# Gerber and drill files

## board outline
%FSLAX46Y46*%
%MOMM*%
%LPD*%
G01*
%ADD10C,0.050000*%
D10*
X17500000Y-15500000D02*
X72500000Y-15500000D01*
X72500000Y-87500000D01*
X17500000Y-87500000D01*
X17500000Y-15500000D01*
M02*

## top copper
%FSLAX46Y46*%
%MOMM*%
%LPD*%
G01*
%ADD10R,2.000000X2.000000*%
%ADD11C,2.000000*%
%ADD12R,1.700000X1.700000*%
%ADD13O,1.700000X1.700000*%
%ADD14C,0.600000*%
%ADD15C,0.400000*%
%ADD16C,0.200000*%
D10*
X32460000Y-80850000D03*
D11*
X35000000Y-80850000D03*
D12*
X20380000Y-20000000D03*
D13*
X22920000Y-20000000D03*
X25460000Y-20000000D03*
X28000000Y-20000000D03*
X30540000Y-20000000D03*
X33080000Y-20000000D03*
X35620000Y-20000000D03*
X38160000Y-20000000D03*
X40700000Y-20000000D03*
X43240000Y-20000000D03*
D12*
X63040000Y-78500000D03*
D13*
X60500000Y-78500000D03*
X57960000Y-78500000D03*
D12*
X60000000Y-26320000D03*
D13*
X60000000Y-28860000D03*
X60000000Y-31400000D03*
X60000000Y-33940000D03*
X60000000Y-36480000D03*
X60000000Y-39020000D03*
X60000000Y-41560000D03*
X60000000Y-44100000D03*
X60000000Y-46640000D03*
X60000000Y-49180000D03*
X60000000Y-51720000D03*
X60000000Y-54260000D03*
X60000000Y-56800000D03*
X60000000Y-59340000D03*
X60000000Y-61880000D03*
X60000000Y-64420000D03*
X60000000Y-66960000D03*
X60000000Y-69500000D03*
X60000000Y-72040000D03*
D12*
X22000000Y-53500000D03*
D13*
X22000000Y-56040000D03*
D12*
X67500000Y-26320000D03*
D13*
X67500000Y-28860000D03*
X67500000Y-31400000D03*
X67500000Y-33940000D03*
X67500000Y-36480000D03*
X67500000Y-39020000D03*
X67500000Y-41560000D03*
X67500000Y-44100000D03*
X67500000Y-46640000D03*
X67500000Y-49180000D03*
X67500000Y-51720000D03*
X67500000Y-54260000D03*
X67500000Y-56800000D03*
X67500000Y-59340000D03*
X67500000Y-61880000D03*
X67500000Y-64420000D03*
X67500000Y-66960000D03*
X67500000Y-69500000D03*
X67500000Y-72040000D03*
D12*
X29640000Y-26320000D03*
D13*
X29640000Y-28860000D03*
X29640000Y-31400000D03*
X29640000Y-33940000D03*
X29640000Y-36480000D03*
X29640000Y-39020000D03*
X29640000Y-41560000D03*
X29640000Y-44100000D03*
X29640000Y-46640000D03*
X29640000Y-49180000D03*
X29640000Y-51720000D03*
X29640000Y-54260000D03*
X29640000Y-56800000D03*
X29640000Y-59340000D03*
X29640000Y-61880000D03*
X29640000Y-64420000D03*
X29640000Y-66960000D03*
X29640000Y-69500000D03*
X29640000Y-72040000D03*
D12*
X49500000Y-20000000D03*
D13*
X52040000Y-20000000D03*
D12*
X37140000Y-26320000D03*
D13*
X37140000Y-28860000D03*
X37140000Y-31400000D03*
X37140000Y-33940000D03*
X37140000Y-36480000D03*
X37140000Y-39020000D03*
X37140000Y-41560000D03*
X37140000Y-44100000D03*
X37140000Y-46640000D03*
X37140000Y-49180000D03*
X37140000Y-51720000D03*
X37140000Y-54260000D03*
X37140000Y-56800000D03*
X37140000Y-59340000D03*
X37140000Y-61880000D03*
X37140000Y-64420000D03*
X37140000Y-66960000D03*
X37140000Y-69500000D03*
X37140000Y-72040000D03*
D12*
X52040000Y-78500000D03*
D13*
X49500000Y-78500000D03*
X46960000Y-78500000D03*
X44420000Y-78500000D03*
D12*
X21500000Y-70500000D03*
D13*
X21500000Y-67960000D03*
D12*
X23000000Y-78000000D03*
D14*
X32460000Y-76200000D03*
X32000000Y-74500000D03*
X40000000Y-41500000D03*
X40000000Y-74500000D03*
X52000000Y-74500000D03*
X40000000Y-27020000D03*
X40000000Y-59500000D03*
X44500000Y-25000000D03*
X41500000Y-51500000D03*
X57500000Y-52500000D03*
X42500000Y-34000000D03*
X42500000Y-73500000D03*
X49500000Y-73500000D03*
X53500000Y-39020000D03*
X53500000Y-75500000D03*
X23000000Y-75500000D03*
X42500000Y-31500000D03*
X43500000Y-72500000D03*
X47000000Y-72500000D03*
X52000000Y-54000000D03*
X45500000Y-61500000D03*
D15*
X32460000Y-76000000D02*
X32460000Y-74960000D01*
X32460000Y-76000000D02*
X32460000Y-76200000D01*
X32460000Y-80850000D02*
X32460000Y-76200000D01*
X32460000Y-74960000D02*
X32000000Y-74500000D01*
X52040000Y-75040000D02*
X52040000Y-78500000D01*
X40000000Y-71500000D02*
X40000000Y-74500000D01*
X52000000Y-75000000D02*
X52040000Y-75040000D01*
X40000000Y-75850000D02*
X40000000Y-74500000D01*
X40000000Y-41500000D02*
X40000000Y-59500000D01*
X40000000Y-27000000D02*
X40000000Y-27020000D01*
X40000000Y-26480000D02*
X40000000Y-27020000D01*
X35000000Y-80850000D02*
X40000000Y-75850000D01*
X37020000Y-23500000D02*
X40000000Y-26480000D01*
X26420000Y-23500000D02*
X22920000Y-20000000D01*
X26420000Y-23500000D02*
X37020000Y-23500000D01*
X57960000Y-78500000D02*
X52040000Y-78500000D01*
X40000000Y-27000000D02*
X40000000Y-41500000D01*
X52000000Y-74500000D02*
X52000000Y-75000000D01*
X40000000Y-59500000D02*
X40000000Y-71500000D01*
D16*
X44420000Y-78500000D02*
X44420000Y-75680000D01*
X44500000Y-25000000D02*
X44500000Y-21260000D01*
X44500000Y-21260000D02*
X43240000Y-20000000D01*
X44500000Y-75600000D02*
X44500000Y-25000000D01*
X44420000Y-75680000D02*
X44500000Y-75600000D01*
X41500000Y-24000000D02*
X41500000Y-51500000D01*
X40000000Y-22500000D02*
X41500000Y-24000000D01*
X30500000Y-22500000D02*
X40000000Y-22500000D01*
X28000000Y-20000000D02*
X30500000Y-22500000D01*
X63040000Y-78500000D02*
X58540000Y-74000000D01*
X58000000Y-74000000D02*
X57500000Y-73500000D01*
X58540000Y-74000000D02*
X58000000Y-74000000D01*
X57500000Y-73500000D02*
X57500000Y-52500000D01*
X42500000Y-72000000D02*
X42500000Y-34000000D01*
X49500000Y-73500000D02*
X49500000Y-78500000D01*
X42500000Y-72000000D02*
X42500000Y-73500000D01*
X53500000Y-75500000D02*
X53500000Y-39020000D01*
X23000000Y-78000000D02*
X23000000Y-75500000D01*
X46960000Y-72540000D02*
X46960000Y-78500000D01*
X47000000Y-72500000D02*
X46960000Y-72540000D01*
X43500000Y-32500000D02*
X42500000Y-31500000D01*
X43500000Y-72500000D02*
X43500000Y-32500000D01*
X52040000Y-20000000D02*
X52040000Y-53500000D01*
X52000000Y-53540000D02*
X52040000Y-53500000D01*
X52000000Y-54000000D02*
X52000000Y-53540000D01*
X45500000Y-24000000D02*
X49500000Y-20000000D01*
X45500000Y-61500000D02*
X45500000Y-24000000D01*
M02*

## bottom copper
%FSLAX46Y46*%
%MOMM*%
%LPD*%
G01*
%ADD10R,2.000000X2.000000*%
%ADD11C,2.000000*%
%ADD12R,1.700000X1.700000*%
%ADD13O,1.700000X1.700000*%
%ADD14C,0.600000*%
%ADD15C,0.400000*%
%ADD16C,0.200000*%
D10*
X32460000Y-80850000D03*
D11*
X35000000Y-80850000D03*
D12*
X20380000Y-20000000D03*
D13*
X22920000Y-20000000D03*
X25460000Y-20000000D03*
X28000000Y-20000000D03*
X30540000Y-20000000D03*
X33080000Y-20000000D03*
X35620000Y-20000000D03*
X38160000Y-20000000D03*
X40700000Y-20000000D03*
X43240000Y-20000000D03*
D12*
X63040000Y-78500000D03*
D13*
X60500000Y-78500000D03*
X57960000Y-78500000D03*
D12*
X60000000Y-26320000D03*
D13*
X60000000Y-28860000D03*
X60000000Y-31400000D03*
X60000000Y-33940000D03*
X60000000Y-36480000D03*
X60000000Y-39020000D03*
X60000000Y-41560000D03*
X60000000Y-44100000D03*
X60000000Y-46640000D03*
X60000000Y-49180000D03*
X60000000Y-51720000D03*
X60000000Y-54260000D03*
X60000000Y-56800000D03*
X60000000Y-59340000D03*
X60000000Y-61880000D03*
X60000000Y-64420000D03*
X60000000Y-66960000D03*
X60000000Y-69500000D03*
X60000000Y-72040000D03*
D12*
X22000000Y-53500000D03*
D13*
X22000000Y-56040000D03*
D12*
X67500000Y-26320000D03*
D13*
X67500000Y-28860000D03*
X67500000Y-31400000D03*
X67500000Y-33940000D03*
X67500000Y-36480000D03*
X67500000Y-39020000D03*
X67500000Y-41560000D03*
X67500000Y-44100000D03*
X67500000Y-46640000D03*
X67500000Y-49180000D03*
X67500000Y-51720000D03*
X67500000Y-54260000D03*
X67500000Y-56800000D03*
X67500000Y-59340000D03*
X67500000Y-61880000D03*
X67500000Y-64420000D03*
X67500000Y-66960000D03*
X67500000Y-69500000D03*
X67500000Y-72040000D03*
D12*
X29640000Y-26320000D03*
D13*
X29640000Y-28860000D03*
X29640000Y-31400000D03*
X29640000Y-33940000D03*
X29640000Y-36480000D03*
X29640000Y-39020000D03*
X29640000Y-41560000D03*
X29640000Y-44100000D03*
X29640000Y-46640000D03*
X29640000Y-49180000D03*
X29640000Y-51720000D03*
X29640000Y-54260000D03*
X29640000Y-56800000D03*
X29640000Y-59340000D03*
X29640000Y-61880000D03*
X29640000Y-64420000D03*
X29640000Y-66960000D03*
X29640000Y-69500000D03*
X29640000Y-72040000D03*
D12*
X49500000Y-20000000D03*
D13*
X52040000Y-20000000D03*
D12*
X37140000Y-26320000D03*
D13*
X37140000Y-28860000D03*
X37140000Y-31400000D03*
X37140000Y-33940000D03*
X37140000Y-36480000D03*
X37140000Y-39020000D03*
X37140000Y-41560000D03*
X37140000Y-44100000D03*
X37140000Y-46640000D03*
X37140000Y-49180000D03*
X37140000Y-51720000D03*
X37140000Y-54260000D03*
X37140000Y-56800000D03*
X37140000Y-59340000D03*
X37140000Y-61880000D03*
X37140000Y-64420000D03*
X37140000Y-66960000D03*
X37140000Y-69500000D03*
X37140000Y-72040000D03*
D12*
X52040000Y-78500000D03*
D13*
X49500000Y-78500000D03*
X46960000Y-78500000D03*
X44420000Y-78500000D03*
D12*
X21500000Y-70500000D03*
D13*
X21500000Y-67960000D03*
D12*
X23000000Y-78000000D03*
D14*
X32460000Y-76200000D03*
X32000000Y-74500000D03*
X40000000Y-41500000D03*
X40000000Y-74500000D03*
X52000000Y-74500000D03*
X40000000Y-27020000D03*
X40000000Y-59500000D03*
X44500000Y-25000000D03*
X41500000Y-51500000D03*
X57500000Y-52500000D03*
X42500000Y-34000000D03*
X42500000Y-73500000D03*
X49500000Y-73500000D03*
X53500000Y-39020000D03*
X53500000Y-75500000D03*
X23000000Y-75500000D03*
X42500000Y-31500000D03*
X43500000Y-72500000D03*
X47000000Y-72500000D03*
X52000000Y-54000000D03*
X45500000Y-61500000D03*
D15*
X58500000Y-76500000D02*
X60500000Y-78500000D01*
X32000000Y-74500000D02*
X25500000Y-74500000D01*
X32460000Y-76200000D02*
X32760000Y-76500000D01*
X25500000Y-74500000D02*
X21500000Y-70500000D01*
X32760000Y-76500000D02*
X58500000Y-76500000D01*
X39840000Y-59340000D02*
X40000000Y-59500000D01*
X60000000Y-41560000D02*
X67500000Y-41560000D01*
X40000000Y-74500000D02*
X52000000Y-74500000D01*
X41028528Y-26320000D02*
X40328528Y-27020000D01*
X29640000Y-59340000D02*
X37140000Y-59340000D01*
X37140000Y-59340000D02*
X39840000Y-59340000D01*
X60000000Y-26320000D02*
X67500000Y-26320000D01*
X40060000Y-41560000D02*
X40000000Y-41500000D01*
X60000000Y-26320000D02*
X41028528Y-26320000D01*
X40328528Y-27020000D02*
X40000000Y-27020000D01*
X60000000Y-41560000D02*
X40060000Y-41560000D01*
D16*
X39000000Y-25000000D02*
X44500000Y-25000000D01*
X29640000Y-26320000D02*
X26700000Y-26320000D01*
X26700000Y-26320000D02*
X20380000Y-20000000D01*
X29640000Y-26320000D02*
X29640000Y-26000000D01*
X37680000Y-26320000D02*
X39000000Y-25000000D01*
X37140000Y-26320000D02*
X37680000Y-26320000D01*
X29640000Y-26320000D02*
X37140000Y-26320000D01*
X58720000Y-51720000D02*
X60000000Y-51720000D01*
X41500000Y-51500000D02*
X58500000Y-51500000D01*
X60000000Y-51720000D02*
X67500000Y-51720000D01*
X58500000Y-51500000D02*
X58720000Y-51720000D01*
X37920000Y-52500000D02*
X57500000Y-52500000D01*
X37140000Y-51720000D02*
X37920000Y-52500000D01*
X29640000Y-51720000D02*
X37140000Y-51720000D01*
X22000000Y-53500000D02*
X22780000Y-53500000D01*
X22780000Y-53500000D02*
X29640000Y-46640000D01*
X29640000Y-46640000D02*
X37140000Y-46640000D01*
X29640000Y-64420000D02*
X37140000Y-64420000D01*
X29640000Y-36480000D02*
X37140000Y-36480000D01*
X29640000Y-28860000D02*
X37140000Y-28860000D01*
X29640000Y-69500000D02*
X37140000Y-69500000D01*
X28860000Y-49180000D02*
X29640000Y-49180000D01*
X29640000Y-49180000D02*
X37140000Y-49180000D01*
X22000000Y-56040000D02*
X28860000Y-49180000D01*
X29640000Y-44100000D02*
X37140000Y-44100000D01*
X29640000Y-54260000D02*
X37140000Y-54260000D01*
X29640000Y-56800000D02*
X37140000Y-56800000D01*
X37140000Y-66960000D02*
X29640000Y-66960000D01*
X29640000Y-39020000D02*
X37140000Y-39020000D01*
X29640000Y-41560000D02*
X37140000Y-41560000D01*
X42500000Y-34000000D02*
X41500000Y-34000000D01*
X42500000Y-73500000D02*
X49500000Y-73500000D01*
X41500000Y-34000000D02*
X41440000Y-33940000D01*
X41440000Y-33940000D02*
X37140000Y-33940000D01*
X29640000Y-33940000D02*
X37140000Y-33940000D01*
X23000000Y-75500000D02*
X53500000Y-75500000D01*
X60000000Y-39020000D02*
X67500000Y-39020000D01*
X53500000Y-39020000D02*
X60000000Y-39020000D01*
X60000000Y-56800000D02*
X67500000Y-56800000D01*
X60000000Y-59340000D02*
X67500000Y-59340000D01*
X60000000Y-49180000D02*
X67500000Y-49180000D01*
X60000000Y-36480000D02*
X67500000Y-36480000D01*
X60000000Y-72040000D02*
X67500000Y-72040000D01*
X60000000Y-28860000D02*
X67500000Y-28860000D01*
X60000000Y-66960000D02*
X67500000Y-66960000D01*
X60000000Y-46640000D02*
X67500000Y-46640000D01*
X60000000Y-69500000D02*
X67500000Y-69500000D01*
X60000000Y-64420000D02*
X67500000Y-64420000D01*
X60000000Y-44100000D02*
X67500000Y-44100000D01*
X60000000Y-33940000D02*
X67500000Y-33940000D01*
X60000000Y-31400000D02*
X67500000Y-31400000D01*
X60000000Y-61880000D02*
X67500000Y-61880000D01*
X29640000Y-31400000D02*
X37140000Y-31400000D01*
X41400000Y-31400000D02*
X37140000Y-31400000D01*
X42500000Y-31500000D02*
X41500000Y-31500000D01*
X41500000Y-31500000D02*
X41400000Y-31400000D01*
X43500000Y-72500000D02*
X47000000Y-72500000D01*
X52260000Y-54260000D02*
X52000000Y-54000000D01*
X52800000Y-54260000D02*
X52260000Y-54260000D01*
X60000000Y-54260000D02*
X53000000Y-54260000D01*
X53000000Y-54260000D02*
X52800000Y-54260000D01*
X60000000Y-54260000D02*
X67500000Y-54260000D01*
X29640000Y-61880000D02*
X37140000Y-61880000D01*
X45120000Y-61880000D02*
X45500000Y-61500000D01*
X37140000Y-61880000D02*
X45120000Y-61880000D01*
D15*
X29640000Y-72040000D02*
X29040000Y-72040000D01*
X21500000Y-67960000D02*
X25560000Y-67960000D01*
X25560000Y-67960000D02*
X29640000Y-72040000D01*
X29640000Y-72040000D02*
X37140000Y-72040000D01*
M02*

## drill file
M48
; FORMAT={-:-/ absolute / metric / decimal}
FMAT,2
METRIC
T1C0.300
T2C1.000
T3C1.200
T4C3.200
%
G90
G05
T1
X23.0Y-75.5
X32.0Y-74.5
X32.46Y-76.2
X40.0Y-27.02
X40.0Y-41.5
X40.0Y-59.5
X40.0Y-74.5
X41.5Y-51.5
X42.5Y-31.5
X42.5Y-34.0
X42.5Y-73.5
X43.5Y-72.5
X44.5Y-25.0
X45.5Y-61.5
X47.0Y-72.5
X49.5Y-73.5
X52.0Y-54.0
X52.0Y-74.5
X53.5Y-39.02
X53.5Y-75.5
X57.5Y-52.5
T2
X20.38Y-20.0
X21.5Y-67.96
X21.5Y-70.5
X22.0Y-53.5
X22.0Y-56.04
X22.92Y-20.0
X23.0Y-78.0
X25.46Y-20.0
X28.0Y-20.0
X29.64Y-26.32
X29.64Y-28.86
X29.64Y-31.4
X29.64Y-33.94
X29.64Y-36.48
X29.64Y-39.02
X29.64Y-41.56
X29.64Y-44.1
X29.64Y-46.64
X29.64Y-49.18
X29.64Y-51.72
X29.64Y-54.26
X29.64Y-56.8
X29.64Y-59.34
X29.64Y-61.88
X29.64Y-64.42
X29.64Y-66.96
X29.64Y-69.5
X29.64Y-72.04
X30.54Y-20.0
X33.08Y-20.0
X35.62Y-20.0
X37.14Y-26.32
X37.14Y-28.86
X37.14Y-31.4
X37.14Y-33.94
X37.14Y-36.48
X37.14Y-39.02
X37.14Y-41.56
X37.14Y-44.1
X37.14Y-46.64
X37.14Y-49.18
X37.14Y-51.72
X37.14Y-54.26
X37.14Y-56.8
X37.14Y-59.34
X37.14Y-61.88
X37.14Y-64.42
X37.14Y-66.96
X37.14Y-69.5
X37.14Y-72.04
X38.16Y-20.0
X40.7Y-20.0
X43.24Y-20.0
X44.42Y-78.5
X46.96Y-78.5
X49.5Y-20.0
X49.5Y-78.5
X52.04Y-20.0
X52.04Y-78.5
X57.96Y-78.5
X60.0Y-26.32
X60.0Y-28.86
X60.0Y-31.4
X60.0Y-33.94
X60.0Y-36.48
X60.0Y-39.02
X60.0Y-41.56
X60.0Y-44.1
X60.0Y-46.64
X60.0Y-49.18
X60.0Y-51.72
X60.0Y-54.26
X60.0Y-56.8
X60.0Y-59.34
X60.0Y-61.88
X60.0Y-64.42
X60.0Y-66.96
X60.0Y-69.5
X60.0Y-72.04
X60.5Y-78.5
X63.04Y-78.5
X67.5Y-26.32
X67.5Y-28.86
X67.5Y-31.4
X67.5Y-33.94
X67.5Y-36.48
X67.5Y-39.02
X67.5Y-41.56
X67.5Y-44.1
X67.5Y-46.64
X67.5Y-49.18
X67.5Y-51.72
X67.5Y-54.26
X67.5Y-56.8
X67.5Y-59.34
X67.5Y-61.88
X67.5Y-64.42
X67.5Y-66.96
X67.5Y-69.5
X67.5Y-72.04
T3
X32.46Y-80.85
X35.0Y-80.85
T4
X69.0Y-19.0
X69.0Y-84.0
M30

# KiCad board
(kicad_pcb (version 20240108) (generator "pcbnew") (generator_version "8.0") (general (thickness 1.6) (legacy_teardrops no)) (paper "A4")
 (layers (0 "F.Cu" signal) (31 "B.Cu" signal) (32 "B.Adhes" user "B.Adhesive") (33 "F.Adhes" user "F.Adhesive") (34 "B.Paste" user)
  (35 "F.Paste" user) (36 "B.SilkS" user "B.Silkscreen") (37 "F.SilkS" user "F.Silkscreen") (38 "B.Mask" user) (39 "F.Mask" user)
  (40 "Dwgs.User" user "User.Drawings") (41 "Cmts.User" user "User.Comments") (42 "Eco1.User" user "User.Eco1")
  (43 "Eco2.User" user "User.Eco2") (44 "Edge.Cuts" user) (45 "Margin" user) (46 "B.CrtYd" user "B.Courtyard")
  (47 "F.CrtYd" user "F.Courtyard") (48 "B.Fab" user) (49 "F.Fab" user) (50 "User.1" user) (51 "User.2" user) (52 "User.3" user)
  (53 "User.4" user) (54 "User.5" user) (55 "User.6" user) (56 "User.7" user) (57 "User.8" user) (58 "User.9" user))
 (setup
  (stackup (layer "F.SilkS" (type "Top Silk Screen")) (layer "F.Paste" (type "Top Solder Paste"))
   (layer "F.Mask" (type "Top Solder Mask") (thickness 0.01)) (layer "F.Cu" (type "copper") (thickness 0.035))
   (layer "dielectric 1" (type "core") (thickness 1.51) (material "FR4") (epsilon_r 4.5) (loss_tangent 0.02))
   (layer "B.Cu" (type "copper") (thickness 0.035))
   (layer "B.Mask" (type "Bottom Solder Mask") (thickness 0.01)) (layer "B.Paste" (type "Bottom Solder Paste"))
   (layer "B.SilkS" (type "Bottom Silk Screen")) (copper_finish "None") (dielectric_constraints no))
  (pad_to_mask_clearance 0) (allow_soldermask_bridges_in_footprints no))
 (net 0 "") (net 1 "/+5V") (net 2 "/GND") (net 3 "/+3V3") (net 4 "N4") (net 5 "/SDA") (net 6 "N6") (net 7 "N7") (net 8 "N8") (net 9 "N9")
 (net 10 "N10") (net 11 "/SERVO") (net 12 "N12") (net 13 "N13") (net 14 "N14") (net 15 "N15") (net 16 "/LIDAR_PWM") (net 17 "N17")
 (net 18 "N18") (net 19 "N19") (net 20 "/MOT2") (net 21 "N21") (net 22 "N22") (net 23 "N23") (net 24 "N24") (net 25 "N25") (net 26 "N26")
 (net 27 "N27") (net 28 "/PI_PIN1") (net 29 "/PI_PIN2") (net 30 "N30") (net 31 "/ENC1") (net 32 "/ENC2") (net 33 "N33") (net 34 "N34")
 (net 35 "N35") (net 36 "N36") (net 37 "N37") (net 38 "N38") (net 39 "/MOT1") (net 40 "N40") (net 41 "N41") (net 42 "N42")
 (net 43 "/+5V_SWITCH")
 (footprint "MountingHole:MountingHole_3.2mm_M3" (layer "F.Cu") (at 69 84)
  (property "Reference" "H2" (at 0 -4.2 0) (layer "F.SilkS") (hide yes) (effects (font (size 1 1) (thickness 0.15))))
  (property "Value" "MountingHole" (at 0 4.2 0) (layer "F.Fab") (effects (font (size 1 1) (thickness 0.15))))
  (pad "" np_thru_hole circle (at 0 0) (size 3.2 3.2) (drill 3.2) (layers "*.Cu" "*.Mask")))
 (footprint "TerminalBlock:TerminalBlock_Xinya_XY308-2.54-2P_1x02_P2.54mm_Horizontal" (layer "F.Cu") (at 32.46 80.85)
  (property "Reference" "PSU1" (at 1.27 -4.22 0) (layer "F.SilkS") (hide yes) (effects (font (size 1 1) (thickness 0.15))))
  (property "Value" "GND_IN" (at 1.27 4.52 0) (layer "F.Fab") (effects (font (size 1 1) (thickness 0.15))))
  (pad "1" thru_hole rect (at 0 0) (size 2 2) (drill 1.2) (layers "*.Cu" "*.Mask") (remove_unused_layers no) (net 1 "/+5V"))
  (pad "2" thru_hole circle (at 2.54 0) (size 2 2) (drill 1.2) (layers "*.Cu" "*.Mask") (remove_unused_layers no) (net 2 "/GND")))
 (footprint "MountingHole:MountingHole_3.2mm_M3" (layer "F.Cu") (at 69 19)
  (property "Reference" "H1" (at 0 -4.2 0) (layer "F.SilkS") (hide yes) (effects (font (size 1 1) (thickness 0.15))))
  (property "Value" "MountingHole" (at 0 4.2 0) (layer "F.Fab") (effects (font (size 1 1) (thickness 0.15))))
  (pad "" np_thru_hole circle (at 0 0) (size 3.2 3.2) (drill 3.2) (layers "*.Cu" "*.Mask")))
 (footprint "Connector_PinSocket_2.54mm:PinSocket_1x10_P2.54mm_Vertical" (layer "F.Cu") (at 20.38 20 90)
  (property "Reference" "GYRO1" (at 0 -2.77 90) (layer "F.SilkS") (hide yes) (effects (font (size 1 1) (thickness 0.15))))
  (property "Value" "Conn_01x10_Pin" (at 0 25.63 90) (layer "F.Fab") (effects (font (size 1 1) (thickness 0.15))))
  (pad "1" thru_hole rect (at 0 0 90) (size 1.7 1.7) (drill 1) (layers "*.Cu" "*.Mask") (remove_unused_layers no) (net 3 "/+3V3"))
  (pad "2" thru_hole oval (at 0 2.54 90) (size 1.7 1.7) (drill 1) (layers "*.Cu" "*.Mask") (remove_unused_layers no) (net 2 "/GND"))
  (pad "3" thru_hole oval (at 0 5.08 90) (size 1.7 1.7) (drill 1) (layers "*.Cu" "*.Mask") (remove_unused_layers no) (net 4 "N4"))
  (pad "4" thru_hole oval (at 0 7.62 90) (size 1.7 1.7) (drill 1) (layers "*.Cu" "*.Mask") (remove_unused_layers no) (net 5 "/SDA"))
  (pad "5" thru_hole oval (at 0 10.16 90) (size 1.7 1.7) (drill 1) (layers "*.Cu" "*.Mask") (remove_unused_layers no) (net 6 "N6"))
  (pad "6" thru_hole oval (at 0 12.7 90) (size 1.7 1.7) (drill 1) (layers "*.Cu" "*.Mask") (remove_unused_layers no) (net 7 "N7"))
  (pad "7" thru_hole oval (at 0 15.24 90) (size 1.7 1.7) (drill 1) (layers "*.Cu" "*.Mask") (remove_unused_layers no) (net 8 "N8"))
  (pad "8" thru_hole oval (at 0 17.78 90) (size 1.7 1.7) (drill 1) (layers "*.Cu" "*.Mask") (remove_unused_layers no) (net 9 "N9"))
  (pad "9" thru_hole oval (at 0 20.32 90) (size 1.7 1.7) (drill 1) (layers "*.Cu" "*.Mask") (remove_unused_layers no) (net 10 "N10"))
  (pad "10" thru_hole oval (at 0 22.86 90) (size 1.7 1.7) (drill 1) (layers "*.Cu" "*.Mask") (remove_unused_layers no) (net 3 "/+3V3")))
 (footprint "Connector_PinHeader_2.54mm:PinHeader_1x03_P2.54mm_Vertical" (layer "F.Cu") (at 63.04 78.5 -90)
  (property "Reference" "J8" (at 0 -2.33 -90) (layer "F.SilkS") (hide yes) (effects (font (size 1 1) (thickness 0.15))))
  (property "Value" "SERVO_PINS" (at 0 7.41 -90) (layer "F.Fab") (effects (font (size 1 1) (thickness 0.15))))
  (pad "1" thru_hole rect (at 0 0 270) (size 1.7 1.7) (drill 1) (layers "*.Cu" "*.Mask") (remove_unused_layers no) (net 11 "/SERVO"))
  (pad "2" thru_hole oval (at 0 2.54 270) (size 1.7 1.7) (drill 1) (layers "*.Cu" "*.Mask") (remove_unused_layers no) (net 1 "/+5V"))
  (pad "3" thru_hole oval (at 0 5.08 270) (size 1.7 1.7) (drill 1) (layers "*.Cu" "*.Mask") (remove_unused_layers no) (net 2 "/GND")))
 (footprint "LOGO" (layer "F.Cu") (at 22.5 37 90)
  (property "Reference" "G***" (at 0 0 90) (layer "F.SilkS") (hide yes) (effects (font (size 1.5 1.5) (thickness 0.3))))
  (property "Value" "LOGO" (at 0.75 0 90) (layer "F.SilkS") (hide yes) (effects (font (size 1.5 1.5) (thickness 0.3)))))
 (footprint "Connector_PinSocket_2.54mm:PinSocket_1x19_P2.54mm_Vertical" (layer "F.Cu") (at 60 26.32)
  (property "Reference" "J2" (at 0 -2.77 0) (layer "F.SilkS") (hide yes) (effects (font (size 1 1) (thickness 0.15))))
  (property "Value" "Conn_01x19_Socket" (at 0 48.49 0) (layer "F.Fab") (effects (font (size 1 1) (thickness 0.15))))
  (pad "1" thru_hole rect (at 0 0) (size 1.7 1.7) (drill 1) (layers "*.Cu" "*.Mask") (remove_unused_layers no) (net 2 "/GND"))
  (pad "2" thru_hole oval (at 0 2.54) (size 1.7 1.7) (drill 1) (layers "*.Cu" "*.Mask") (remove_unused_layers no) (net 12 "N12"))
  (pad "3" thru_hole oval (at 0 5.08) (size 1.7 1.7) (drill 1) (layers "*.Cu" "*.Mask") (remove_unused_layers no) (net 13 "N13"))
  (pad "4" thru_hole oval (at 0 7.62) (size 1.7 1.7) (drill 1) (layers "*.Cu" "*.Mask") (remove_unused_layers no) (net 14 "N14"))
  (pad "5" thru_hole oval (at 0 10.16) (size 1.7 1.7) (drill 1) (layers "*.Cu" "*.Mask") (remove_unused_layers no) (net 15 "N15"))
  (pad "6" thru_hole oval (at 0 12.7) (size 1.7 1.7) (drill 1) (layers "*.Cu" "*.Mask") (remove_unused_layers no) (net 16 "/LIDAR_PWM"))
  (pad "7" thru_hole oval (at 0 15.24) (size 1.7 1.7) (drill 1) (layers "*.Cu" "*.Mask") (remove_unused_layers no) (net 2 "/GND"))
  (pad "8" thru_hole oval (at 0 17.78) (size 1.7 1.7) (drill 1) (layers "*.Cu" "*.Mask") (remove_unused_layers no) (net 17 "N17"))
  (pad "9" thru_hole oval (at 0 20.32) (size 1.7 1.7) (drill 1) (layers "*.Cu" "*.Mask") (remove_unused_layers no) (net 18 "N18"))
  (pad "10" thru_hole oval (at 0 22.86) (size 1.7 1.7) (drill 1) (layers "*.Cu" "*.Mask") (remove_unused_layers no) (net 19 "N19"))
  (pad "11" thru_hole oval (at 0 25.4) (size 1.7 1.7) (drill 1) (layers "*.Cu" "*.Mask") (remove_unused_layers no) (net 5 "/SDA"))
  (pad "12" thru_hole oval (at 0 27.94) (size 1.7 1.7) (drill 1) (layers "*.Cu" "*.Mask") (remove_unused_layers no) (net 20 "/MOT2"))
  (pad "13" thru_hole oval (at 0 30.48) (size 1.7 1.7) (drill 1) (layers "*.Cu" "*.Mask") (remove_unused_layers no) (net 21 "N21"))
  (pad "14" thru_hole oval (at 0 33.02) (size 1.7 1.7) (drill 1) (layers "*.Cu" "*.Mask") (remove_unused_layers no) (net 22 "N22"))
  (pad "15" thru_hole oval (at 0 35.56) (size 1.7 1.7) (drill 1) (layers "*.Cu" "*.Mask") (remove_unused_layers no) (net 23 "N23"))
  (pad "16" thru_hole oval (at 0 38.1) (size 1.7 1.7) (drill 1) (layers "*.Cu" "*.Mask") (remove_unused_layers no) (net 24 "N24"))
  (pad "17" thru_hole oval (at 0 40.64) (size 1.7 1.7) (drill 1) (layers "*.Cu" "*.Mask") (remove_unused_layers no) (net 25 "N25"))
  (pad "18" thru_hole oval (at 0 43.18) (size 1.7 1.7) (drill 1) (layers "*.Cu" "*.Mask") (remove_unused_layers no) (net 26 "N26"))
  (pad "19" thru_hole oval (at 0 45.72) (size 1.7 1.7) (drill 1) (layers "*.Cu" "*.Mask") (remove_unused_layers no) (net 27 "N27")))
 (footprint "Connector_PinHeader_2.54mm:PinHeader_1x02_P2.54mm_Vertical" (layer "F.Cu") (at 22 53.5)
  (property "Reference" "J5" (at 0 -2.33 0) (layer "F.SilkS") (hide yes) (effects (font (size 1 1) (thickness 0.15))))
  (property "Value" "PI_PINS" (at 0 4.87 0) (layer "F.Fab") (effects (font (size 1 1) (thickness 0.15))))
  (pad "1" thru_hole rect (at 0 0) (size 1.7 1.7) (drill 1) (layers "*.Cu" "*.Mask") (remove_unused_layers no) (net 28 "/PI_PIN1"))
  (pad "2" thru_hole oval (at 0 2.54) (size 1.7 1.7) (drill 1) (layers "*.Cu" "*.Mask") (remove_unused_layers no) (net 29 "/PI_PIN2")))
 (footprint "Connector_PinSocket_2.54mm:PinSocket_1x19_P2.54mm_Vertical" (layer "F.Cu") (at 67.5 26.32)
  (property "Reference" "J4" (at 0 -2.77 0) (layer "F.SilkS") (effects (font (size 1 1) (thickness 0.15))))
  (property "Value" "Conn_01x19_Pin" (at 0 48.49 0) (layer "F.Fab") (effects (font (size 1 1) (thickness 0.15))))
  (pad "1" thru_hole rect (at 0 0) (size 1.7 1.7) (drill 1) (layers "*.Cu" "*.Mask") (remove_unused_layers no) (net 2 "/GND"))
  (pad "2" thru_hole oval (at 0 2.54) (size 1.7 1.7) (drill 1) (layers "*.Cu" "*.Mask") (remove_unused_layers no) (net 12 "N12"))
  (pad "3" thru_hole oval (at 0 5.08) (size 1.7 1.7) (drill 1) (layers "*.Cu" "*.Mask") (remove_unused_layers no) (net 13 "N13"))
  (pad "4" thru_hole oval (at 0 7.62) (size 1.7 1.7) (drill 1) (layers "*.Cu" "*.Mask") (remove_unused_layers no) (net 14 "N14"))
  (pad "5" thru_hole oval (at 0 10.16) (size 1.7 1.7) (drill 1) (layers "*.Cu" "*.Mask") (remove_unused_layers no) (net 15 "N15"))
  (pad "6" thru_hole oval (at 0 12.7) (size 1.7 1.7) (drill 1) (layers "*.Cu" "*.Mask") (remove_unused_layers no) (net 16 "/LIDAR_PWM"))
  (pad "7" thru_hole oval (at 0 15.24) (size 1.7 1.7) (drill 1) (layers "*.Cu" "*.Mask") (remove_unused_layers no) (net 2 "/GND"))
  (pad "8" thru_hole oval (at 0 17.78) (size 1.7 1.7) (drill 1) (layers "*.Cu" "*.Mask") (remove_unused_layers no) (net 17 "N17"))
  (pad "9" thru_hole oval (at 0 20.32) (size 1.7 1.7) (drill 1) (layers "*.Cu" "*.Mask") (remove_unused_layers no) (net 18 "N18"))
  (pad "10" thru_hole oval (at 0 22.86) (size 1.7 1.7) (drill 1) (layers "*.Cu" "*.Mask") (remove_unused_layers no) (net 19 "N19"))
  (pad "11" thru_hole oval (at 0 25.4) (size 1.7 1.7) (drill 1) (layers "*.Cu" "*.Mask") (remove_unused_layers no) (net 5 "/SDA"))
  (pad "12" thru_hole oval (at 0 27.94) (size 1.7 1.7) (drill 1) (layers "*.Cu" "*.Mask") (remove_unused_layers no) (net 20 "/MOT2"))
  (pad "13" thru_hole oval (at 0 30.48) (size 1.7 1.7) (drill 1) (layers "*.Cu" "*.Mask") (remove_unused_layers no) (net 21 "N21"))
  (pad "14" thru_hole oval (at 0 33.02) (size 1.7 1.7) (drill 1) (layers "*.Cu" "*.Mask") (remove_unused_layers no) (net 22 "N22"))
  (pad "15" thru_hole oval (at 0 35.56) (size 1.7 1.7) (drill 1) (layers "*.Cu" "*.Mask") (remove_unused_layers no) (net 23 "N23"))
  (pad "16" thru_hole oval (at 0 38.1) (size 1.7 1.7) (drill 1) (layers "*.Cu" "*.Mask") (remove_unused_layers no) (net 24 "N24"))
  (pad "17" thru_hole oval (at 0 40.64) (size 1.7 1.7) (drill 1) (layers "*.Cu" "*.Mask") (remove_unused_layers no) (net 25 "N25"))
  (pad "18" thru_hole oval (at 0 43.18) (size 1.7 1.7) (drill 1) (layers "*.Cu" "*.Mask") (remove_unused_layers no) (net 26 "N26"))
  (pad "19" thru_hole oval (at 0 45.72) (size 1.7 1.7) (drill 1) (layers "*.Cu" "*.Mask") (remove_unused_layers no) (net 27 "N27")))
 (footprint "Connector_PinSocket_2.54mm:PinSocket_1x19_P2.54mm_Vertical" (layer "F.Cu") (at 29.64 26.32)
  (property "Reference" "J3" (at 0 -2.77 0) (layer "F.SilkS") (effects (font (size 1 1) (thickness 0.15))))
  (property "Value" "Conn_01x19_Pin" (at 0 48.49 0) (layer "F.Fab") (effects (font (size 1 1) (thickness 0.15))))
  (pad "1" thru_hole rect (at 0 0) (size 1.7 1.7) (drill 1) (layers "*.Cu" "*.Mask") (remove_unused_layers no) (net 3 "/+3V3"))
  (pad "2" thru_hole oval (at 0 2.54) (size 1.7 1.7) (drill 1) (layers "*.Cu" "*.Mask") (remove_unused_layers no) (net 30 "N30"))
  (pad "3" thru_hole oval (at 0 5.08) (size 1.7 1.7) (drill 1) (layers "*.Cu" "*.Mask") (remove_unused_layers no) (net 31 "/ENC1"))
  (pad "4" thru_hole oval (at 0 7.62) (size 1.7 1.7) (drill 1) (layers "*.Cu" "*.Mask") (remove_unused_layers no) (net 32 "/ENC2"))
  (pad "5" thru_hole oval (at 0 10.16) (size 1.7 1.7) (drill 1) (layers "*.Cu" "*.Mask") (remove_unused_layers no) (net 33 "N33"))
  (pad "6" thru_hole oval (at 0 12.7) (size 1.7 1.7) (drill 1) (layers "*.Cu" "*.Mask") (remove_unused_layers no) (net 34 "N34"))
  (pad "7" thru_hole oval (at 0 15.24) (size 1.7 1.7) (drill 1) (layers "*.Cu" "*.Mask") (remove_unused_layers no) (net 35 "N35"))
  (pad "8" thru_hole oval (at 0 17.78) (size 1.7 1.7) (drill 1) (layers "*.Cu" "*.Mask") (remove_unused_layers no) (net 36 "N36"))
  (pad "9" thru_hole oval (at 0 20.32) (size 1.7 1.7) (drill 1) (layers "*.Cu" "*.Mask") (remove_unused_layers no) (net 28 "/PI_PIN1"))
  (pad "10" thru_hole oval (at 0 22.86) (size 1.7 1.7) (drill 1) (layers "*.Cu" "*.Mask") (remove_unused_layers no) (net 29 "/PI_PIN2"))
  (pad "11" thru_hole oval (at 0 25.4) (size 1.7 1.7) (drill 1) (layers "*.Cu" "*.Mask") (remove_unused_layers no) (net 11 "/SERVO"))
  (pad "12" thru_hole oval (at 0 27.94) (size 1.7 1.7) (drill 1) (layers "*.Cu" "*.Mask") (remove_unused_layers no) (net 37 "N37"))
  (pad "13" thru_hole oval (at 0 30.48) (size 1.7 1.7) (drill 1) (layers "*.Cu" "*.Mask") (remove_unused_layers no) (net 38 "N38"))
  (pad "14" thru_hole oval (at 0 33.02) (size 1.7 1.7) (drill 1) (layers "*.Cu" "*.Mask") (remove_unused_layers no) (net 2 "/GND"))
  (pad "15" thru_hole oval (at 0 35.56) (size 1.7 1.7) (drill 1) (layers "*.Cu" "*.Mask") (remove_unused_layers no) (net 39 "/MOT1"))
  (pad "16" thru_hole oval (at 0 38.1) (size 1.7 1.7) (drill 1) (layers "*.Cu" "*.Mask") (remove_unused_layers no) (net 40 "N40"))
  (pad "17" thru_hole oval (at 0 40.64) (size 1.7 1.7) (drill 1) (layers "*.Cu" "*.Mask") (remove_unused_layers no) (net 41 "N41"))
  (pad "18" thru_hole oval (at 0 43.18) (size 1.7 1.7) (drill 1) (layers "*.Cu" "*.Mask") (remove_unused_layers no) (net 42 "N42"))
  (pad "19" thru_hole oval (at 0 45.72) (size 1.7 1.7) (drill 1) (layers "*.Cu" "*.Mask") (remove_unused_layers no) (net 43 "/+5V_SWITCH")))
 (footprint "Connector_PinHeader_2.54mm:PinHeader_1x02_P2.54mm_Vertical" (layer "F.Cu") (at 49.5 20 90)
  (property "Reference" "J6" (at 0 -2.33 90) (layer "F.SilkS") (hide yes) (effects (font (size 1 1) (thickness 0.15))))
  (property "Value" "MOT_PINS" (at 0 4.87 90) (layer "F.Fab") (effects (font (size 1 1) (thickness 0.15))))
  (pad "1" thru_hole rect (at 0 0 90) (size 1.7 1.7) (drill 1) (layers "*.Cu" "*.Mask") (remove_unused_layers no) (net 39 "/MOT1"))
  (pad "2" thru_hole oval (at 0 2.54 90) (size 1.7 1.7) (drill 1) (layers "*.Cu" "*.Mask") (remove_unused_layers no) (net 20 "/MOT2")))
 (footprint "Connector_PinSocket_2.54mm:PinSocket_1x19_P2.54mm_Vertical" (layer "F.Cu") (at 37.14 26.32)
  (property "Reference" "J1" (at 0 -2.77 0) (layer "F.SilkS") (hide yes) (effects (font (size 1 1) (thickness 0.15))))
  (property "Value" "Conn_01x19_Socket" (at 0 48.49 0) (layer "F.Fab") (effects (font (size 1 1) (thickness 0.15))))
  (pad "1" thru_hole rect (at 0 0) (size 1.7 1.7) (drill 1) (layers "*.Cu" "*.Mask") (remove_unused_layers no) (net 3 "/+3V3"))
  (pad "2" thru_hole oval (at 0 2.54) (size 1.7 1.7) (drill 1) (layers "*.Cu" "*.Mask") (remove_unused_layers no) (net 30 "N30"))
  (pad "3" thru_hole oval (at 0 5.08) (size 1.7 1.7) (drill 1) (layers "*.Cu" "*.Mask") (remove_unused_layers no) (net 31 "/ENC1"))
  (pad "4" thru_hole oval (at 0 7.62) (size 1.7 1.7) (drill 1) (layers "*.Cu" "*.Mask") (remove_unused_layers no) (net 32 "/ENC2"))
  (pad "5" thru_hole oval (at 0 10.16) (size 1.7 1.7) (drill 1) (layers "*.Cu" "*.Mask") (remove_unused_layers no) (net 33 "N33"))
  (pad "6" thru_hole oval (at 0 12.7) (size 1.7 1.7) (drill 1) (layers "*.Cu" "*.Mask") (remove_unused_layers no) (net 34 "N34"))
  (pad "7" thru_hole oval (at 0 15.24) (size 1.7 1.7) (drill 1) (layers "*.Cu" "*.Mask") (remove_unused_layers no) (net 35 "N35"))
  (pad "8" thru_hole oval (at 0 17.78) (size 1.7 1.7) (drill 1) (layers "*.Cu" "*.Mask") (remove_unused_layers no) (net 36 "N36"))
  (pad "9" thru_hole oval (at 0 20.32) (size 1.7 1.7) (drill 1) (layers "*.Cu" "*.Mask") (remove_unused_layers no) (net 28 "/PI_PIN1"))
  (pad "10" thru_hole oval (at 0 22.86) (size 1.7 1.7) (drill 1) (layers "*.Cu" "*.Mask") (remove_unused_layers no) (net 29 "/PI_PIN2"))
  (pad "11" thru_hole oval (at 0 25.4) (size 1.7 1.7) (drill 1) (layers "*.Cu" "*.Mask") (remove_unused_layers no) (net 11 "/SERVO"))
  (pad "12" thru_hole oval (at 0 27.94) (size 1.7 1.7) (drill 1) (layers "*.Cu" "*.Mask") (remove_unused_layers no) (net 37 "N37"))
  (pad "13" thru_hole oval (at 0 30.48) (size 1.7 1.7) (drill 1) (layers "*.Cu" "*.Mask") (remove_unused_layers no) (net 38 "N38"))
  (pad "14" thru_hole oval (at 0 33.02) (size 1.7 1.7) (drill 1) (layers "*.Cu" "*.Mask") (remove_unused_layers no) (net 2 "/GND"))
  (pad "15" thru_hole oval (at 0 35.56) (size 1.7 1.7) (drill 1) (layers "*.Cu" "*.Mask") (remove_unused_layers no) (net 39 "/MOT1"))
  (pad "16" thru_hole oval (at 0 38.1) (size 1.7 1.7) (drill 1) (layers "*.Cu" "*.Mask") (remove_unused_layers no) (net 40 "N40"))
  (pad "17" thru_hole oval (at 0 40.64) (size 1.7 1.7) (drill 1) (layers "*.Cu" "*.Mask") (remove_unused_layers no) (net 41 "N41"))
  (pad "18" thru_hole oval (at 0 43.18) (size 1.7 1.7) (drill 1) (layers "*.Cu" "*.Mask") (remove_unused_layers no) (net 42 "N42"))
  (pad "19" thru_hole oval (at 0 45.72) (size 1.7 1.7) (drill 1) (layers "*.Cu" "*.Mask") (remove_unused_layers no) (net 43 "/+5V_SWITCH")))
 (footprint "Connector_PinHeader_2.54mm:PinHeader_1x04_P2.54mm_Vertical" (layer "F.Cu") (at 52.04 78.5 -90)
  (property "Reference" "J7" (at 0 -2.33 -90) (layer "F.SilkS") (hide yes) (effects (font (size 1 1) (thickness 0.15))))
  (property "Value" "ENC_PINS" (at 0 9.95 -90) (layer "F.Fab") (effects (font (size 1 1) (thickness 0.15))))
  (pad "1" thru_hole rect (at 0 0 270) (size 1.7 1.7) (drill 1) (layers "*.Cu" "*.Mask") (remove_unused_layers no) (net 2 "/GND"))
  (pad "2" thru_hole oval (at 0 2.54 270) (size 1.7 1.7) (drill 1) (layers "*.Cu" "*.Mask") (remove_unused_layers no) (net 32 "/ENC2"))
  (pad "3" thru_hole oval (at 0 5.08 270) (size 1.7 1.7) (drill 1) (layers "*.Cu" "*.Mask") (remove_unused_layers no) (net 31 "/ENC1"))
  (pad "4" thru_hole oval (at 0 7.62 270) (size 1.7 1.7) (drill 1) (layers "*.Cu" "*.Mask") (remove_unused_layers no) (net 3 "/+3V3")))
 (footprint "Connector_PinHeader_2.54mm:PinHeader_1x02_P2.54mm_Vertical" (layer "F.Cu") (at 21.5 70.5 180)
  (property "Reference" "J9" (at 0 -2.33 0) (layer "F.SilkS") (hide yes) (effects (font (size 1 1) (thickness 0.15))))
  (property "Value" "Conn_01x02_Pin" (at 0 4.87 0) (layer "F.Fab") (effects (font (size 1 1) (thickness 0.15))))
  (pad "1" thru_hole rect (at 0 0 180) (size 1.7 1.7) (drill 1) (layers "*.Cu" "*.Mask") (remove_unused_layers no) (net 1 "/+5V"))
  (pad "2" thru_hole oval (at 0 2.54 180) (size 1.7 1.7) (drill 1) (layers "*.Cu" "*.Mask") (remove_unused_layers no) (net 43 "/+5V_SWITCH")))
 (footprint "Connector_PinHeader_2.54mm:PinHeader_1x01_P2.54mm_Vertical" (layer "F.Cu") (at 23 78 -90)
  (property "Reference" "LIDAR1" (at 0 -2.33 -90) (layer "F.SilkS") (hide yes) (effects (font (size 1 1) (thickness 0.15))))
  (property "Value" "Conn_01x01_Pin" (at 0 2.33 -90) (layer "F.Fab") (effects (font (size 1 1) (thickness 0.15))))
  (pad "1" thru_hole rect (at 0 0 270) (size 1.7 1.7) (drill 1) (layers "*.Cu" "*.Mask") (remove_unused_layers no) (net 16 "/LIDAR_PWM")))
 (gr_rect (start 17.5 15.5) (end 72.5 87.5) (stroke (width 0.05) (type default)) (fill none) (layer "Edge.Cuts"))
 (segment (start 32.46 76) (end 32.46 74.96) (width 0.4) (layer "F.Cu") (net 1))
 (segment (start 32.46 76) (end 32.46 76.2) (width 0.4) (layer "F.Cu") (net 1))
 (segment (start 32.46 80.85) (end 32.46 76.2) (width 0.4) (layer "F.Cu") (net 1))
 (segment (start 32.46 74.96) (end 32 74.5) (width 0.4) (layer "F.Cu") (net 1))
 (via (at 32.46 76.2) (size 0.6) (drill 0.3) (layers "F.Cu" "B.Cu") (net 1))
 (via (at 32 74.5) (size 0.6) (drill 0.3) (layers "F.Cu" "B.Cu") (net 1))
 (segment (start 58.5 76.5) (end 60.5 78.5) (width 0.4) (layer "B.Cu") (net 1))
 (segment (start 32 74.5) (end 25.5 74.5) (width 0.4) (layer "B.Cu") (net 1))
 (segment (start 32.46 76.2) (end 32.76 76.5) (width 0.4) (layer "B.Cu") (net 1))
 (segment (start 25.5 74.5) (end 21.5 70.5) (width 0.4) (layer "B.Cu") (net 1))
 (segment (start 32.76 76.5) (end 58.5 76.5) (width 0.4) (layer "B.Cu") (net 1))
 (segment (start 52.04 75.04) (end 52.04 78.5) (width 0.4) (layer "F.Cu") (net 2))
 (segment (start 40 71.5) (end 40 74.5) (width 0.4) (layer "F.Cu") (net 2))
 (segment (start 52 75) (end 52.04 75.04) (width 0.4) (layer "F.Cu") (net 2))
 (segment (start 40 75.85) (end 40 74.5) (width 0.4) (layer "F.Cu") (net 2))
 (segment (start 40 41.5) (end 40 59.5) (width 0.4) (layer "F.Cu") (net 2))
 (segment (start 40 27) (end 40 27.02) (width 0.4) (layer "F.Cu") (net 2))
 (segment (start 40 26.48) (end 40 27.02) (width 0.4) (layer "F.Cu") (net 2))
 (segment (start 35 80.85) (end 40 75.85) (width 0.4) (layer "F.Cu") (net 2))
 (segment (start 37.02 23.5) (end 40 26.48) (width 0.4) (layer "F.Cu") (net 2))
 (segment (start 26.42 23.5) (end 22.92 20) (width 0.4) (layer "F.Cu") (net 2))
 (segment (start 26.42 23.5) (end 37.02 23.5) (width 0.4) (layer "F.Cu") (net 2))
 (segment (start 57.96 78.5) (end 52.04 78.5) (width 0.4) (layer "F.Cu") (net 2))
 (segment (start 40 27) (end 40 41.5) (width 0.4) (layer "F.Cu") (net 2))
 (segment (start 52 74.5) (end 52 75) (width 0.4) (layer "F.Cu") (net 2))
 (segment (start 40 59.5) (end 40 71.5) (width 0.4) (layer "F.Cu") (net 2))
 (via (at 40 41.5) (size 0.6) (drill 0.3) (layers "F.Cu" "B.Cu") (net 2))
 (via (at 40 74.5) (size 0.6) (drill 0.3) (layers "F.Cu" "B.Cu") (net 2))
 (via (at 52 74.5) (size 0.6) (drill 0.3) (layers "F.Cu" "B.Cu") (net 2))
 (via (at 40 27.02) (size 0.6) (drill 0.3) (layers "F.Cu" "B.Cu") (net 2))
 (via (at 40 59.5) (size 0.6) (drill 0.3) (layers "F.Cu" "B.Cu") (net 2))
 (segment (start 39.84 59.34) (end 40 59.5) (width 0.4) (layer "B.Cu") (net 2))
 (segment (start 60 41.56) (end 67.5 41.56) (width 0.4) (layer "B.Cu") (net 2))
 (segment (start 40 74.5) (end 52 74.5) (width 0.4) (layer "B.Cu") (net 2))
 (segment (start 41.028528 26.32) (end 40.328528 27.02) (width 0.4) (layer "B.Cu") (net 2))
 (segment (start 29.64 59.34) (end 37.14 59.34) (width 0.4) (layer "B.Cu") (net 2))
 (segment (start 37.14 59.34) (end 39.84 59.34) (width 0.4) (layer "B.Cu") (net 2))
 (segment (start 60 26.32) (end 67.5 26.32) (width 0.4) (layer "B.Cu") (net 2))
 (segment (start 40.06 41.56) (end 40 41.5) (width 0.4) (layer "B.Cu") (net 2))
 (segment (start 60 26.32) (end 41.028528 26.32) (width 0.4) (layer "B.Cu") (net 2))
 (segment (start 40.328528 27.02) (end 40 27.02) (width 0.4) (layer "B.Cu") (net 2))
 (segment (start 60 41.56) (end 40.06 41.56) (width 0.4) (layer "B.Cu") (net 2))
 (segment (start 44.42 78.5) (end 44.42 75.68) (width 0.2) (layer "F.Cu") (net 3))
 (segment (start 44.5 25) (end 44.5 21.26) (width 0.2) (layer "F.Cu") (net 3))
 (segment (start 44.5 21.26) (end 43.24 20) (width 0.2) (layer "F.Cu") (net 3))
 (segment (start 44.5 75.6) (end 44.5 25) (width 0.2) (layer "F.Cu") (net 3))
 (segment (start 44.42 75.68) (end 44.5 75.6) (width 0.2) (layer "F.Cu") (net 3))
 (via (at 44.5 25) (size 0.6) (drill 0.3) (layers "F.Cu" "B.Cu") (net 3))
 (segment (start 39 25) (end 44.5 25) (width 0.2) (layer "B.Cu") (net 3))
 (segment (start 29.64 26.32) (end 26.7 26.32) (width 0.2) (layer "B.Cu") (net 3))
 (segment (start 26.7 26.32) (end 20.38 20) (width 0.2) (layer "B.Cu") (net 3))
 (segment (start 29.64 26.32) (end 29.64 26) (width 0.2) (layer "B.Cu") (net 3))
 (segment (start 37.68 26.32) (end 39 25) (width 0.2) (layer "B.Cu") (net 3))
 (segment (start 37.14 26.32) (end 37.68 26.32) (width 0.2) (layer "B.Cu") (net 3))
 (segment (start 29.64 26.32) (end 37.14 26.32) (width 0.2) (layer "B.Cu") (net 3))
 (segment (start 41.5 24) (end 41.5 51.5) (width 0.2) (layer "F.Cu") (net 5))
 (segment (start 40 22.5) (end 41.5 24) (width 0.2) (layer "F.Cu") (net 5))
 (segment (start 30.5 22.5) (end 40 22.5) (width 0.2) (layer "F.Cu") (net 5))
 (segment (start 28 20) (end 30.5 22.5) (width 0.2) (layer "F.Cu") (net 5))
 (via (at 41.5 51.5) (size 0.6) (drill 0.3) (layers "F.Cu" "B.Cu") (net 5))
 (segment (start 58.72 51.72) (end 60 51.72) (width 0.2) (layer "B.Cu") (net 5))
 (segment (start 41.5 51.5) (end 58.5 51.5) (width 0.2) (layer "B.Cu") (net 5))
 (segment (start 60 51.72) (end 67.5 51.72) (width 0.2) (layer "B.Cu") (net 5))
 (segment (start 58.5 51.5) (end 58.72 51.72) (width 0.2) (layer "B.Cu") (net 5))
 (segment (start 63.04 78.5) (end 58.54 74) (width 0.2) (layer "F.Cu") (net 11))
 (segment (start 58 74) (end 57.5 73.5) (width 0.2) (layer "F.Cu") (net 11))
 (segment (start 58.54 74) (end 58 74) (width 0.2) (layer "F.Cu") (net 11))
 (segment (start 57.5 73.5) (end 57.5 52.5) (width 0.2) (layer "F.Cu") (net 11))
 (via (at 57.5 52.5) (size 0.6) (drill 0.3) (layers "F.Cu" "B.Cu") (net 11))
 (segment (start 37.92 52.5) (end 57.5 52.5) (width 0.2) (layer "B.Cu") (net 11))
 (segment (start 37.14 51.72) (end 37.92 52.5) (width 0.2) (layer "B.Cu") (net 11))
 (segment (start 29.64 51.72) (end 37.14 51.72) (width 0.2) (layer "B.Cu") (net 11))
 (segment (start 22 53.5) (end 22.78 53.5) (width 0.2) (layer "B.Cu") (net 28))
 (segment (start 22.78 53.5) (end 29.64 46.64) (width 0.2) (layer "B.Cu") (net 28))
 (segment (start 29.64 46.64) (end 37.14 46.64) (width 0.2) (layer "B.Cu") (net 28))
 (segment (start 29.64 64.42) (end 37.14 64.42) (width 0.2) (layer "B.Cu") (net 40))
 (segment (start 29.64 36.48) (end 37.14 36.48) (width 0.2) (layer "B.Cu") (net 33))
 (segment (start 29.64 28.86) (end 37.14 28.86) (width 0.2) (layer "B.Cu") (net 30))
 (segment (start 29.64 69.5) (end 37.14 69.5) (width 0.2) (layer "B.Cu") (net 42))
 (segment (start 28.86 49.18) (end 29.64 49.18) (width 0.2) (layer "B.Cu") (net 29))
 (segment (start 29.64 49.18) (end 37.14 49.18) (width 0.2) (layer "B.Cu") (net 29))
 (segment (start 22 56.04) (end 28.86 49.18) (width 0.2) (layer "B.Cu") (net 29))
 (segment (start 29.64 44.1) (end 37.14 44.1) (width 0.2) (layer "B.Cu") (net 36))
 (segment (start 29.64 54.26) (end 37.14 54.26) (width 0.2) (layer "B.Cu") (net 37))
 (segment (start 29.64 56.8) (end 37.14 56.8) (width 0.2) (layer "B.Cu") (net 38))
 (segment (start 37.14 66.96) (end 29.64 66.96) (width 0.2) (layer "B.Cu") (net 41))
 (segment (start 29.64 39.02) (end 37.14 39.02) (width 0.2) (layer "B.Cu") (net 34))
 (segment (start 29.64 41.56) (end 37.14 41.56) (width 0.2) (layer "B.Cu") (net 35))
 (segment (start 42.5 72) (end 42.5 34) (width 0.2) (layer "F.Cu") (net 32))
 (segment (start 49.5 73.5) (end 49.5 78.5) (width 0.2) (layer "F.Cu") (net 32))
 (segment (start 42.5 72) (end 42.5 73.5) (width 0.2) (layer "F.Cu") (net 32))
 (via (at 42.5 34) (size 0.6) (drill 0.3) (layers "F.Cu" "B.Cu") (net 32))
 (via (at 42.5 73.5) (size 0.6) (drill 0.3) (layers "F.Cu" "B.Cu") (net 32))
 (via (at 49.5 73.5) (size 0.6) (drill 0.3) (layers "F.Cu" "B.Cu") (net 32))
 (segment (start 42.5 34) (end 41.5 34) (width 0.2) (layer "B.Cu") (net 32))
 (segment (start 42.5 73.5) (end 49.5 73.5) (width 0.2) (layer "B.Cu") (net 32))
 (segment (start 41.5 34) (end 41.44 33.94) (width 0.2) (layer "B.Cu") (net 32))
 (segment (start 41.44 33.94) (end 37.14 33.94) (width 0.2) (layer "B.Cu") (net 32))
 (segment (start 29.64 33.94) (end 37.14 33.94) (width 0.2) (layer "B.Cu") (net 32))
 (segment (start 53.5 75.5) (end 53.5 39.02) (width 0.2) (layer "F.Cu") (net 16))
 (segment (start 23 78) (end 23 75.5) (width 0.2) (layer "F.Cu") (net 16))
 (via (at 53.5 39.02) (size 0.6) (drill 0.3) (layers "F.Cu" "B.Cu") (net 16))
 (via (at 53.5 75.5) (size 0.6) (drill 0.3) (layers "F.Cu" "B.Cu") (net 16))
 (via (at 23 75.5) (size 0.6) (drill 0.3) (layers "F.Cu" "B.Cu") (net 16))
 (segment (start 23 75.5) (end 53.5 75.5) (width 0.2) (layer "B.Cu") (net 16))
 (segment (start 60 39.02) (end 67.5 39.02) (width 0.2) (layer "B.Cu") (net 16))
 (segment (start 53.5 39.02) (end 60 39.02) (width 0.2) (layer "B.Cu") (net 16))
 (segment (start 60 56.8) (end 67.5 56.8) (width 0.2) (layer "B.Cu") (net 21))
 (segment (start 60 59.34) (end 67.5 59.34) (width 0.2) (layer "B.Cu") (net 22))
 (segment (start 60 49.18) (end 67.5 49.18) (width 0.2) (layer "B.Cu") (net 19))
 (segment (start 60 36.48) (end 67.5 36.48) (width 0.2) (layer "B.Cu") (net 15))
 (segment (start 60 72.04) (end 67.5 72.04) (width 0.2) (layer "B.Cu") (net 27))
 (segment (start 60 28.86) (end 67.5 28.86) (width 0.2) (layer "B.Cu") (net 12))
 (segment (start 60 66.96) (end 67.5 66.96) (width 0.2) (layer "B.Cu") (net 25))
 (segment (start 60 46.64) (end 67.5 46.64) (width 0.2) (layer "B.Cu") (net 18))
 (segment (start 60 69.5) (end 67.5 69.5) (width 0.2) (layer "B.Cu") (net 26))
 (segment (start 60 64.42) (end 67.5 64.42) (width 0.2) (layer "B.Cu") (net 24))
 (segment (start 60 44.1) (end 67.5 44.1) (width 0.2) (layer "B.Cu") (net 17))
 (segment (start 60 33.94) (end 67.5 33.94) (width 0.2) (layer "B.Cu") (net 14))
 (segment (start 60 31.4) (end 67.5 31.4) (width 0.2) (layer "B.Cu") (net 13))
 (segment (start 60 61.88) (end 67.5 61.88) (width 0.2) (layer "B.Cu") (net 23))
 (segment (start 46.96 72.54) (end 46.96 78.5) (width 0.2) (layer "F.Cu") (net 31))
 (segment (start 47 72.5) (end 46.96 72.54) (width 0.2) (layer "F.Cu") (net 31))
 (segment (start 43.5 32.5) (end 42.5 31.5) (width 0.2) (layer "F.Cu") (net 31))
 (segment (start 43.5 72.5) (end 43.5 32.5) (width 0.2) (layer "F.Cu") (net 31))
 (via (at 42.5 31.5) (size 0.6) (drill 0.3) (layers "F.Cu" "B.Cu") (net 31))
 (via (at 43.5 72.5) (size 0.6) (drill 0.3) (layers "F.Cu" "B.Cu") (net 31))
 (via (at 47 72.5) (size 0.6) (drill 0.3) (layers "F.Cu" "B.Cu") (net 31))
 (segment (start 29.64 31.4) (end 37.14 31.4) (width 0.2) (layer "B.Cu") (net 31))
 (segment (start 41.4 31.4) (end 37.14 31.4) (width 0.2) (layer "B.Cu") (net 31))
 (segment (start 42.5 31.5) (end 41.5 31.5) (width 0.2) (layer "B.Cu") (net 31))
 (segment (start 41.5 31.5) (end 41.4 31.4) (width 0.2) (layer "B.Cu") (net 31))
 (segment (start 43.5 72.5) (end 47 72.5) (width 0.2) (layer "B.Cu") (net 31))
 (segment (start 52.04 20) (end 52.04 53.5) (width 0.2) (layer "F.Cu") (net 20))
 (segment (start 52 53.54) (end 52.04 53.5) (width 0.2) (layer "F.Cu") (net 20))
 (segment (start 52 54) (end 52 53.54) (width 0.2) (layer "F.Cu") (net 20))
 (via (at 52 54) (size 0.6) (drill 0.3) (layers "F.Cu" "B.Cu") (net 20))
 (segment (start 52.26 54.26) (end 52 54) (width 0.2) (layer "B.Cu") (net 20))
 (segment (start 52.8 54.26) (end 52.26 54.26) (width 0.2) (layer "B.Cu") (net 20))
 (segment (start 60 54.26) (end 53 54.26) (width 0.2) (layer "B.Cu") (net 20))
 (segment (start 53 54.26) (end 52.8 54.26) (width 0.2) (layer "B.Cu") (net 20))
 (segment (start 60 54.26) (end 67.5 54.26) (width 0.2) (layer "B.Cu") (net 20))
 (segment (start 45.5 24) (end 49.5 20) (width 0.2) (layer "F.Cu") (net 39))
 (segment (start 45.5 61.5) (end 45.5 24) (width 0.2) (layer "F.Cu") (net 39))
 (via (at 45.5 61.5) (size 0.6) (drill 0.3) (layers "F.Cu" "B.Cu") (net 39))
 (segment (start 29.64 61.88) (end 37.14 61.88) (width 0.2) (layer "B.Cu") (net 39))
 (segment (start 45.12 61.88) (end 45.5 61.5) (width 0.2) (layer "B.Cu") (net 39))
 (segment (start 37.14 61.88) (end 45.12 61.88) (width 0.2) (layer "B.Cu") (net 39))
 (segment (start 29.64 72.04) (end 29.04 72.04) (width 0.4) (layer "B.Cu") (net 43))
 (segment (start 21.5 67.96) (end 25.56 67.96) (width 0.4) (layer "B.Cu") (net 43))
 (segment (start 25.56 67.96) (end 29.64 72.04) (width 0.4) (layer "B.Cu") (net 43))
 (segment (start 29.64 72.04) (end 37.14 72.04) (width 0.4) (layer "B.Cu") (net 43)))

